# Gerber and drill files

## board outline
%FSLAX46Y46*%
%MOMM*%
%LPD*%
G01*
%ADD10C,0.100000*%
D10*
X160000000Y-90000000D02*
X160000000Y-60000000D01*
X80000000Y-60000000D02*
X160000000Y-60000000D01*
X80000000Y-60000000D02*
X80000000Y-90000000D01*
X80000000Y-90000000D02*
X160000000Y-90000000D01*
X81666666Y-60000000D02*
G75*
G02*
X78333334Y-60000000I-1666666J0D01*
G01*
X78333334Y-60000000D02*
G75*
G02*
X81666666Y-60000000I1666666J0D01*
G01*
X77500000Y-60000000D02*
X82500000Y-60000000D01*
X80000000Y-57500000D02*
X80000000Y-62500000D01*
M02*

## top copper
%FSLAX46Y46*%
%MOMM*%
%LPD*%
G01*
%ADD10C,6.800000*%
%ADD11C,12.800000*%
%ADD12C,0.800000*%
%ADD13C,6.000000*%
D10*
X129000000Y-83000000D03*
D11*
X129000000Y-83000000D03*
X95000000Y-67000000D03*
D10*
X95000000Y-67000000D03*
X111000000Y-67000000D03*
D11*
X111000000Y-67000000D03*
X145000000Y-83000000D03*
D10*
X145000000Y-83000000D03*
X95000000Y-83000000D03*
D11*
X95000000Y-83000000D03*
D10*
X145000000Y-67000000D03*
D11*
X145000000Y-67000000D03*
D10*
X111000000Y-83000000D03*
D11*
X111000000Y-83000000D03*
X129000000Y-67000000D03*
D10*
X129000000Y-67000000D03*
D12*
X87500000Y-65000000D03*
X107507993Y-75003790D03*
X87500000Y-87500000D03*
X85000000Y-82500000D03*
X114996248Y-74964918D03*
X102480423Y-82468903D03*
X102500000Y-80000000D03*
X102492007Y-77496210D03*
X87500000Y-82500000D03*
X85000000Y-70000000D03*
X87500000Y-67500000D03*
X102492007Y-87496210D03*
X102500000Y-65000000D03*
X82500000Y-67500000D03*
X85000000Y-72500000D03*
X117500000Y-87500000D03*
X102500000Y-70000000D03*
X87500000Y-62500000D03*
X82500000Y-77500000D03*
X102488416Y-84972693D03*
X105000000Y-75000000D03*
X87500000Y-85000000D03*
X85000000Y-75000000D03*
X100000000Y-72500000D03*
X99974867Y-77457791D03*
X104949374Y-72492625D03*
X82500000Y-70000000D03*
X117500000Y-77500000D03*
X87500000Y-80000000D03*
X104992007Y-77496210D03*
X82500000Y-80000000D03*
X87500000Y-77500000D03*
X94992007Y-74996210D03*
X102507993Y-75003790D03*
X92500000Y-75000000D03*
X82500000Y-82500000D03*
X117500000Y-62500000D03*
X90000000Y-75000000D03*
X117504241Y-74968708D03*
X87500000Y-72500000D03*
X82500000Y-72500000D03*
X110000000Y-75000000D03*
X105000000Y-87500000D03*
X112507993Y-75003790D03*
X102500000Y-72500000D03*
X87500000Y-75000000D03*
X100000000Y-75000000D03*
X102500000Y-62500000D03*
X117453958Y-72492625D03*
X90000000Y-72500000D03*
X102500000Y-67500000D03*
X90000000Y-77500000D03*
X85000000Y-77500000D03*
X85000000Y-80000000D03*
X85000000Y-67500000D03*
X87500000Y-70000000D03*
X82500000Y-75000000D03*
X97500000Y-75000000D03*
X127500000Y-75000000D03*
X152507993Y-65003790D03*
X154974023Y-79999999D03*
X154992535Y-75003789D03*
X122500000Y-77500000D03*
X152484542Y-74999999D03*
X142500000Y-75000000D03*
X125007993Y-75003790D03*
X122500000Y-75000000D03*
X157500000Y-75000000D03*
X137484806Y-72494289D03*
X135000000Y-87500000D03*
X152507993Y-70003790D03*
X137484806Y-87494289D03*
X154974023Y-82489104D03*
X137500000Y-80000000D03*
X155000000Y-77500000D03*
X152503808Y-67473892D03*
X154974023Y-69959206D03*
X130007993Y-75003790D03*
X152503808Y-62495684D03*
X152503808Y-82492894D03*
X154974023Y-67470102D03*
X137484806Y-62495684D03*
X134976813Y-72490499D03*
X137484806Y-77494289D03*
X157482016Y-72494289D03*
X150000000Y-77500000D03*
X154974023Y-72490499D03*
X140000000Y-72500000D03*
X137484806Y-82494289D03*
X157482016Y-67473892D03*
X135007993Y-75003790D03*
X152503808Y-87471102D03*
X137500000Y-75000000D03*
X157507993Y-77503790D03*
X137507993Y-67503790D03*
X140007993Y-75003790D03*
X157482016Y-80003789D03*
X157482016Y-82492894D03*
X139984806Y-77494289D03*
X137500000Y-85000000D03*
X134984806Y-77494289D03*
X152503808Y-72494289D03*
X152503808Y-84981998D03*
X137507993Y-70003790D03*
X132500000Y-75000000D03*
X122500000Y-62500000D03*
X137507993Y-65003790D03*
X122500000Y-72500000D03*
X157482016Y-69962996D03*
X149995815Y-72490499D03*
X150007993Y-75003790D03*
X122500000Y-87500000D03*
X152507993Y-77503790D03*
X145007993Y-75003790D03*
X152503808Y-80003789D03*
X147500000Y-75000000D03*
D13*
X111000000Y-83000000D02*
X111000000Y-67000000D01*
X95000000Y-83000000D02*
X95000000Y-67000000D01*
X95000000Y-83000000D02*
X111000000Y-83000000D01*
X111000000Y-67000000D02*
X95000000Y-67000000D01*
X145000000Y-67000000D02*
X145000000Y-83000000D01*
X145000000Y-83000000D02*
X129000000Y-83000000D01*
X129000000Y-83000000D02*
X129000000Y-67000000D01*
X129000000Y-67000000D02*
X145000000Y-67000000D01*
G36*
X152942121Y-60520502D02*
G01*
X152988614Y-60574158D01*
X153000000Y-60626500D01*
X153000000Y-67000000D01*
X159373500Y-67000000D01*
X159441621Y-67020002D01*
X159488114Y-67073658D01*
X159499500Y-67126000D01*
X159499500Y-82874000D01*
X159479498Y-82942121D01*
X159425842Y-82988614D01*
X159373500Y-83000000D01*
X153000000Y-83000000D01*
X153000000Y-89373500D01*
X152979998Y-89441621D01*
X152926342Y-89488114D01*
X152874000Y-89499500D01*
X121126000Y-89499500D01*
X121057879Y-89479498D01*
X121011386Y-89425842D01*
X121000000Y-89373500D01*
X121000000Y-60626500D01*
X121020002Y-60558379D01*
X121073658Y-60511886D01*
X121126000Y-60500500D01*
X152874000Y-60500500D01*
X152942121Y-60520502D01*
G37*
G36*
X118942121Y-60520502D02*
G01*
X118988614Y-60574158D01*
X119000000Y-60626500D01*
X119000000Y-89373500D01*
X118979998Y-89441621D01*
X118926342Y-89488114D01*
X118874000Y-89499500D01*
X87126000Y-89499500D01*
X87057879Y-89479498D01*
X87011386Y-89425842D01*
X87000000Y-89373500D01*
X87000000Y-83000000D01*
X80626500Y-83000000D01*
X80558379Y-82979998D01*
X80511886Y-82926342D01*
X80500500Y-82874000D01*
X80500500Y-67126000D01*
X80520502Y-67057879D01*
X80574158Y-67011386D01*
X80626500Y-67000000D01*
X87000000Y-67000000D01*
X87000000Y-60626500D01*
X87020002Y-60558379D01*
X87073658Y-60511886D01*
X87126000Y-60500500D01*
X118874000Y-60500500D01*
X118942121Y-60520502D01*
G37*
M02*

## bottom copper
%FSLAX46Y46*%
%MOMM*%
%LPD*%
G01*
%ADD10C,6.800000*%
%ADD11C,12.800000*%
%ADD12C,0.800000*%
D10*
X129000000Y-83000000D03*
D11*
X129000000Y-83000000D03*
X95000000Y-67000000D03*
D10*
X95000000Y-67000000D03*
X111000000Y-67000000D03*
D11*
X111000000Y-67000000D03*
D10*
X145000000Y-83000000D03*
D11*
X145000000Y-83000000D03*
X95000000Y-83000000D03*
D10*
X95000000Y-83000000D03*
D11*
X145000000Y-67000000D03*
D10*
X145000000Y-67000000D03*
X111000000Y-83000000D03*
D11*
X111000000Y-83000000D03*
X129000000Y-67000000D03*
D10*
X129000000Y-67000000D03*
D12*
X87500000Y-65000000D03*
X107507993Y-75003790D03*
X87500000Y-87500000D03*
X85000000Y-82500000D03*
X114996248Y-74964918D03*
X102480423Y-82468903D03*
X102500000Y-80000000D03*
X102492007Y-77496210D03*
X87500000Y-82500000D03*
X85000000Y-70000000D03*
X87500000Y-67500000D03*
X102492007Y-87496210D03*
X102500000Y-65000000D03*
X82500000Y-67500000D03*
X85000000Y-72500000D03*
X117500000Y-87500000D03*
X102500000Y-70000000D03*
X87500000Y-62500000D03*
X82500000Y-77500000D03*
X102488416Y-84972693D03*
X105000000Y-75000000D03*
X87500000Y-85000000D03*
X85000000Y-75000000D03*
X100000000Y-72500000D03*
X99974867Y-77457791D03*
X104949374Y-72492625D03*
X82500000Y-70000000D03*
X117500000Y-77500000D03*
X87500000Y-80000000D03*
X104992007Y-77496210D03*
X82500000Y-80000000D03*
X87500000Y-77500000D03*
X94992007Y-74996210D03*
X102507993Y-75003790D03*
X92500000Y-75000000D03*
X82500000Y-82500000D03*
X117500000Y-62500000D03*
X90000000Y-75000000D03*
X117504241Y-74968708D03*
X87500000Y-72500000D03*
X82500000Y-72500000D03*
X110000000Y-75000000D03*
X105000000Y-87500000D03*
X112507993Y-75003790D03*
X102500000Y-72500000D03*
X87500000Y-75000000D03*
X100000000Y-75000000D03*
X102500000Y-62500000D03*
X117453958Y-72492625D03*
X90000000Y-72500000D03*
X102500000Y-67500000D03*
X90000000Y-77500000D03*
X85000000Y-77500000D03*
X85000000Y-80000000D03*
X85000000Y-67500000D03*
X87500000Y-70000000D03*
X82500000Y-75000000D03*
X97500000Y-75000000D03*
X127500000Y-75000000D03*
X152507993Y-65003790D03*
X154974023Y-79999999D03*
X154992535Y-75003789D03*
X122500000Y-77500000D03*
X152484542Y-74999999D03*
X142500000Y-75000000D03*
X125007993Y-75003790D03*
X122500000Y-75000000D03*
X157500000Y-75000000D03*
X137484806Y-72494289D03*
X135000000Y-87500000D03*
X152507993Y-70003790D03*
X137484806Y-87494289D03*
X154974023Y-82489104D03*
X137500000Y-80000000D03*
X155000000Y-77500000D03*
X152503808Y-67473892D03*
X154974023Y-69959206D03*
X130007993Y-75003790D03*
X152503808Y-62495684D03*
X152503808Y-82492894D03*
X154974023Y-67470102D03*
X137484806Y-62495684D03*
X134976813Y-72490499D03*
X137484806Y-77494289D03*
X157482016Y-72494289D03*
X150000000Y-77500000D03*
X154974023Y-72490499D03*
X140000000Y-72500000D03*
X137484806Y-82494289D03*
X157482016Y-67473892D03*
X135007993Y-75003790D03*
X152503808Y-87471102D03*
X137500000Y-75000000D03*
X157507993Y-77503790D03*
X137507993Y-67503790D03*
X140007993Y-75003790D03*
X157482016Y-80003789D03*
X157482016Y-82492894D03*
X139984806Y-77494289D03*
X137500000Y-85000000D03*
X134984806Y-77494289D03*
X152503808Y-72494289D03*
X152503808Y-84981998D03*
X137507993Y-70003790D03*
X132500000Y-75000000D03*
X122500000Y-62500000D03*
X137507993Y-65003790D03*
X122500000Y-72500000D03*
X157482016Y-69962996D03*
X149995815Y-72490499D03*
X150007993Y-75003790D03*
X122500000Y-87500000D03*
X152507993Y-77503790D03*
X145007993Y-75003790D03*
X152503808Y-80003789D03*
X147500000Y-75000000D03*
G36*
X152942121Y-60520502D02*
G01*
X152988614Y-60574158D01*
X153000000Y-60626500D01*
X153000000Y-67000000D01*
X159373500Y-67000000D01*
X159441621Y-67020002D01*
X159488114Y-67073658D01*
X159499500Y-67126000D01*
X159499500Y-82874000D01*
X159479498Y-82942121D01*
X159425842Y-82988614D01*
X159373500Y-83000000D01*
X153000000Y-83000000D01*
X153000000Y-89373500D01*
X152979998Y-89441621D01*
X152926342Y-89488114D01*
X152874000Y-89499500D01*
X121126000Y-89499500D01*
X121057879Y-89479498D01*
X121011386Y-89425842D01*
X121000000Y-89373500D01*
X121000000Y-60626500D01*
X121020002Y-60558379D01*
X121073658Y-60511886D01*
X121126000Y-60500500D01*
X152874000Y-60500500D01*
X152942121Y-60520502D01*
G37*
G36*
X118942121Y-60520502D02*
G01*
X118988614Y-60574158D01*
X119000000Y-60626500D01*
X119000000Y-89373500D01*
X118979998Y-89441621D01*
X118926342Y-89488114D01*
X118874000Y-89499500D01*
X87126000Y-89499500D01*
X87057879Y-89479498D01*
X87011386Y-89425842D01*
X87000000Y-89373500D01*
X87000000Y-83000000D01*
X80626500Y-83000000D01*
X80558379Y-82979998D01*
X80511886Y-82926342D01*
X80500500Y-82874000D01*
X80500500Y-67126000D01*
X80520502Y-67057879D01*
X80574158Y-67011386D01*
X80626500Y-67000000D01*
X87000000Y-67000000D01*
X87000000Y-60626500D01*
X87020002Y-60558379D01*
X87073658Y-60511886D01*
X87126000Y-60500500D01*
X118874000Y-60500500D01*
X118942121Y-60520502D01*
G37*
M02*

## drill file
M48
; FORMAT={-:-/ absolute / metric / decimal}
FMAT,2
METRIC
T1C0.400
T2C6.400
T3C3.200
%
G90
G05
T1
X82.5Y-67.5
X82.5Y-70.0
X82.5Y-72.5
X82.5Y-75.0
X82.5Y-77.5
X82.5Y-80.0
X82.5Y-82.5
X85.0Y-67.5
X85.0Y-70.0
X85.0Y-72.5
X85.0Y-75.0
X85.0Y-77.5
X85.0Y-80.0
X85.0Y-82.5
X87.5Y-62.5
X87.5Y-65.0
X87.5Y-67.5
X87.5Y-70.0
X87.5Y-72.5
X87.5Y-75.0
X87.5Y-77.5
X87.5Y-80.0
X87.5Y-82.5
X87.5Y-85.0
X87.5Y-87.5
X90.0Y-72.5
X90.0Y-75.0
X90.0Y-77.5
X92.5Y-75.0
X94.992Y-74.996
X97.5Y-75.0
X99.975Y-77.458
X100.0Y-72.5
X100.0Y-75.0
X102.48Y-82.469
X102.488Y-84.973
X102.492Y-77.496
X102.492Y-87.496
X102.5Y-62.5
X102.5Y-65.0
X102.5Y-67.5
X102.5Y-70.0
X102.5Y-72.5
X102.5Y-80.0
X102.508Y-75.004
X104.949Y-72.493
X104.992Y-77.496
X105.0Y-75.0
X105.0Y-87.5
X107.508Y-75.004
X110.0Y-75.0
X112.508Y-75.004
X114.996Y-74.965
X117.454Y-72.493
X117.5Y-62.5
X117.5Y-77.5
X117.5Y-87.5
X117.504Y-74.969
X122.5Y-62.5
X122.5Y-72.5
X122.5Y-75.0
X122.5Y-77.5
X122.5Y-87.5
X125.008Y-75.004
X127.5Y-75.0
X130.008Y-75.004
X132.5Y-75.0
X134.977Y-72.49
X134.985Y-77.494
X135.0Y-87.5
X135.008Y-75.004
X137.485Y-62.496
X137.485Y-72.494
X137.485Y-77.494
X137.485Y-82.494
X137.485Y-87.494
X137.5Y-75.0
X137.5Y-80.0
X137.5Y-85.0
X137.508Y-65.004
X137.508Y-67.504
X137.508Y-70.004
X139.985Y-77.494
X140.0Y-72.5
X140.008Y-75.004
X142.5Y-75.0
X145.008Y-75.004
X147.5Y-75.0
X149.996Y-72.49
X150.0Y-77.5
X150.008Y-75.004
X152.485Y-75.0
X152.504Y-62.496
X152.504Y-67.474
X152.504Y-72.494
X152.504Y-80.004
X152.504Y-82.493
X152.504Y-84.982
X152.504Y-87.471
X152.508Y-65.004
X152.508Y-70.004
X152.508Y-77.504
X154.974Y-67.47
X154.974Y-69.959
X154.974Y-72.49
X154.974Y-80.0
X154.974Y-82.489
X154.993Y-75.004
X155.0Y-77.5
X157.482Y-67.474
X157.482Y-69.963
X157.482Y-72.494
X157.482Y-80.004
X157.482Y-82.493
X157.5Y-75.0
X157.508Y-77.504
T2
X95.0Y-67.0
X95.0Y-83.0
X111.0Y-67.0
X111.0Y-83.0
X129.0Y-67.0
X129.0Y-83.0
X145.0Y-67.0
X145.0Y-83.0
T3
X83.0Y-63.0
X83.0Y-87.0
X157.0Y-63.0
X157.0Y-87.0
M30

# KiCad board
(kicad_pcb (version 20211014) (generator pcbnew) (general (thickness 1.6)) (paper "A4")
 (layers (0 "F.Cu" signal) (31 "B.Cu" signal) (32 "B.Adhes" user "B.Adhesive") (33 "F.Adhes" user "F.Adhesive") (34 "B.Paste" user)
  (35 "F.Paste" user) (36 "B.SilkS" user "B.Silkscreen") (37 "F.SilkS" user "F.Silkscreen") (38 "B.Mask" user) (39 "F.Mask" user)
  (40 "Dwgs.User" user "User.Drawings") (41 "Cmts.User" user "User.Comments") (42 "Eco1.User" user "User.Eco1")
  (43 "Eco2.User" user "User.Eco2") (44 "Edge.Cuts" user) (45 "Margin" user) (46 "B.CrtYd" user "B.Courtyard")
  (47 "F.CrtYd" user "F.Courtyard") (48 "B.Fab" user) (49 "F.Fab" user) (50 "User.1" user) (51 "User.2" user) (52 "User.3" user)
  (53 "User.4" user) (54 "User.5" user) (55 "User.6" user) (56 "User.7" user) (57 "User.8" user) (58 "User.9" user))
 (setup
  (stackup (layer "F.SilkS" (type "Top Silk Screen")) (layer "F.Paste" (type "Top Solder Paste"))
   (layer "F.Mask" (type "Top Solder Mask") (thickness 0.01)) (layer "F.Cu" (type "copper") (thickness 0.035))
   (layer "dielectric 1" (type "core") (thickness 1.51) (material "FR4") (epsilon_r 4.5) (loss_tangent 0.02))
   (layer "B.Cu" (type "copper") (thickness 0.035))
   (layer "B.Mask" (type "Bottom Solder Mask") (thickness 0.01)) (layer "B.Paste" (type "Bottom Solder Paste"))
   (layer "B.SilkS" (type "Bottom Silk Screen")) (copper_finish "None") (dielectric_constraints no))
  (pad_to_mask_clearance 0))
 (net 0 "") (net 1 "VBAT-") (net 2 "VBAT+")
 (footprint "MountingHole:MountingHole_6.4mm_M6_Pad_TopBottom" (layer "F.Cu") (at 129 83 90)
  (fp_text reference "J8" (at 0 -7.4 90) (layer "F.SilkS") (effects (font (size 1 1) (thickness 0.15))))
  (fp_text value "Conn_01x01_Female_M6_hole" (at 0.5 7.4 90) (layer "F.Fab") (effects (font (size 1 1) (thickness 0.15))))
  (pad "1" thru_hole circle locked (at 0 0 90) (size 6.8 6.8) (drill 6.4) (layers *.Cu *.Mask) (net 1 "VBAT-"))
  (pad "1" connect circle locked (at 0 0 90) (size 12.8 12.8) (layers "F.Cu" "F.Mask") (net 1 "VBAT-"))
  (pad "1" connect circle locked (at 0 0 90) (size 12.8 12.8) (layers "B.Cu" "B.Mask") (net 1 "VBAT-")))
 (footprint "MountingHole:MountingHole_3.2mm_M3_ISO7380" (layer "F.Cu") (at 157 87)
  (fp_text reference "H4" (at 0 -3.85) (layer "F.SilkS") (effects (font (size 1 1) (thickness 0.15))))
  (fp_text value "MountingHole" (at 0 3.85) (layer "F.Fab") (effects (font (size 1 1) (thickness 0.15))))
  (pad "" np_thru_hole circle locked (at 0 0) (size 3.2 3.2) (drill 3.2) (layers *.Cu *.Mask)))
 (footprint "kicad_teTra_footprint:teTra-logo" (layer "F.Cu") (at 85 74 -90)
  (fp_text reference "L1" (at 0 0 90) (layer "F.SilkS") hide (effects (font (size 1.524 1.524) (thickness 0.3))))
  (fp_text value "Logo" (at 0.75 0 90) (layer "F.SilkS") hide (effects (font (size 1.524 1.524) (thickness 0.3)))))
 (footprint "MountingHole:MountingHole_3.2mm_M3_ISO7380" (layer "F.Cu") (at 83 87)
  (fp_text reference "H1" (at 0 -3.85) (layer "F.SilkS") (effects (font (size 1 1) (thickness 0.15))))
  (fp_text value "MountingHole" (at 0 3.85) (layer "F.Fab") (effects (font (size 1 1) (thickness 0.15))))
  (pad "" np_thru_hole circle locked (at 0 0) (size 3.2 3.2) (drill 3.2) (layers *.Cu *.Mask)))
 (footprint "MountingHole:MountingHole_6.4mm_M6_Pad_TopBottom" (layer "F.Cu") (at 95 67 90)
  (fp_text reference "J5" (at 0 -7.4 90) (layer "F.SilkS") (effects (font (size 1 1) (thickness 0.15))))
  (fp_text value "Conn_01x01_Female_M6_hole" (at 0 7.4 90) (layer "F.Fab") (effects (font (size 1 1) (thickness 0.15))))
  (pad "1" connect circle locked (at 0 0 90) (size 12.8 12.8) (layers "B.Cu" "B.Mask") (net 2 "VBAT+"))
  (pad "1" connect circle locked (at 0 0 90) (size 12.8 12.8) (layers "F.Cu" "F.Mask") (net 2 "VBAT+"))
  (pad "1" thru_hole circle locked (at 0 0 90) (size 6.8 6.8) (drill 6.4) (layers *.Cu *.Mask) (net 2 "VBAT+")))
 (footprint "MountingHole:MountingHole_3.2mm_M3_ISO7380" (layer "F.Cu") (at 83 63)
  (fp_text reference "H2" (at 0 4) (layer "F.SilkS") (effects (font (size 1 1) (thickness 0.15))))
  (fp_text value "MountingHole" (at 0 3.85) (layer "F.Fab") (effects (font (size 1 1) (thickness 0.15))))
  (pad "" np_thru_hole circle locked (at 0 0) (size 3.2 3.2) (drill 3.2) (layers *.Cu *.Mask)))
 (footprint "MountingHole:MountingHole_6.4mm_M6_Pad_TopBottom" (layer "F.Cu") (at 111 67 90)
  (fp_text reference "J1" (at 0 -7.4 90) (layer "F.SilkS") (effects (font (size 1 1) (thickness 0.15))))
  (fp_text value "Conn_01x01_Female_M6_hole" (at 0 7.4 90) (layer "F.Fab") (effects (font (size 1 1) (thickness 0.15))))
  (pad "1" thru_hole circle locked (at 0 0 90) (size 6.8 6.8) (drill 6.4) (layers *.Cu *.Mask) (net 2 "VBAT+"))
  (pad "1" connect circle locked (at 0 0 90) (size 12.8 12.8) (layers "F.Cu" "F.Mask") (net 2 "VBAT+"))
  (pad "1" connect circle locked (at 0 0 90) (size 12.8 12.8) (layers "B.Cu" "B.Mask") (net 2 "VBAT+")))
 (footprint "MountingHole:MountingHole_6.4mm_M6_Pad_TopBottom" (layer "F.Cu") (at 145 83 90)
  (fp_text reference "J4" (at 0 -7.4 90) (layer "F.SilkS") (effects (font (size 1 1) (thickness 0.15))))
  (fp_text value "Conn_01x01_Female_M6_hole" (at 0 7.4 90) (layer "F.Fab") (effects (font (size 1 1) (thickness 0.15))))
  (pad "1" connect circle locked (at 0 0 90) (size 12.8 12.8) (layers "F.Cu" "F.Mask") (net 1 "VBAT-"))
  (pad "1" thru_hole circle locked (at 0 0 90) (size 6.8 6.8) (drill 6.4) (layers *.Cu *.Mask) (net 1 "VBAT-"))
  (pad "1" connect circle locked (at 0 0 90) (size 12.8 12.8) (layers "B.Cu" "B.Mask") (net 1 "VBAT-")))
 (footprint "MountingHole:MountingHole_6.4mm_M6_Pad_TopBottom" (layer "F.Cu") (at 95 83 90)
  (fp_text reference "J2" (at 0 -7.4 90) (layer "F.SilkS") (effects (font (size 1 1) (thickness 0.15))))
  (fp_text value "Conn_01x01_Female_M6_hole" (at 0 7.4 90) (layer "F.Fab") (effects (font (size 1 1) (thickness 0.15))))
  (pad "1" connect circle locked (at 0 0 90) (size 12.8 12.8) (layers "B.Cu" "B.Mask") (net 2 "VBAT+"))
  (pad "1" thru_hole circle locked (at 0 0 90) (size 6.8 6.8) (drill 6.4) (layers *.Cu *.Mask) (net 2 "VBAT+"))
  (pad "1" connect circle locked (at 0 0 90) (size 12.8 12.8) (layers "F.Cu" "F.Mask") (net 2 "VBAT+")))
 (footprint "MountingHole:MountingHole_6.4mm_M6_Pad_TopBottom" (layer "F.Cu") (at 145 67 90)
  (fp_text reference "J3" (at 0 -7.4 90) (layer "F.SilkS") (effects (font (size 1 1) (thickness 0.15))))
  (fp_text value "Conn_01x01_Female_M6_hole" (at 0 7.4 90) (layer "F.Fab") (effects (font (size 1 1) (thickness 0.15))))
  (pad "1" connect circle locked (at 0 0 90) (size 12.8 12.8) (layers "B.Cu" "B.Mask") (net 1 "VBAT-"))
  (pad "1" thru_hole circle locked (at 0 0 90) (size 6.8 6.8) (drill 6.4) (layers *.Cu *.Mask) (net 1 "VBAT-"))
  (pad "1" connect circle locked (at 0 0 90) (size 12.8 12.8) (layers "F.Cu" "F.Mask") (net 1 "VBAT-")))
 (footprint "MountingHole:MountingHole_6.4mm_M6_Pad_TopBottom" (layer "F.Cu") (at 111 83 90)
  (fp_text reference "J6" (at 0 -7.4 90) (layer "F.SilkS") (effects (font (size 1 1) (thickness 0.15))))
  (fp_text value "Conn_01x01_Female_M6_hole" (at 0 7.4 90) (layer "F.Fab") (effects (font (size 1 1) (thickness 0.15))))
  (pad "1" thru_hole circle locked (at 0 0 90) (size 6.8 6.8) (drill 6.4) (layers *.Cu *.Mask) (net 2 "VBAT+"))
  (pad "1" connect circle locked (at 0 0 90) (size 12.8 12.8) (layers "B.Cu" "B.Mask") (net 2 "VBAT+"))
  (pad "1" connect circle locked (at 0 0 90) (size 12.8 12.8) (layers "F.Cu" "F.Mask") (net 2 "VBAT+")))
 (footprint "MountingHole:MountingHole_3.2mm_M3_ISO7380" (layer "F.Cu") (at 157 63)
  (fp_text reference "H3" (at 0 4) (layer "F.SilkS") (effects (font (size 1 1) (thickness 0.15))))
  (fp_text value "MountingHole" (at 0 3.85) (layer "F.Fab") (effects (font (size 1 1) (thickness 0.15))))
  (pad "" np_thru_hole circle locked (at 0 0) (size 3.2 3.2) (drill 3.2) (layers *.Cu *.Mask)))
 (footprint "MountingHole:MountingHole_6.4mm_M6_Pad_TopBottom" (layer "F.Cu") (at 129 67 90)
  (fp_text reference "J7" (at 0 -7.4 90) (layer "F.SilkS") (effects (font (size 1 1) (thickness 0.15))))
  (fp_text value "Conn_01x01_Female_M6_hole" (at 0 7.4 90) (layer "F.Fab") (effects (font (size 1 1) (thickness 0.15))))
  (pad "1" connect circle locked (at 0 0 90) (size 12.8 12.8) (layers "F.Cu" "F.Mask") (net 1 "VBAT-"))
  (pad "1" connect circle locked (at 0 0 90) (size 12.8 12.8) (layers "B.Cu" "B.Mask") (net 1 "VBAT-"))
  (pad "1" thru_hole circle locked (at 0 0 90) (size 6.8 6.8) (drill 6.4) (layers *.Cu *.Mask) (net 1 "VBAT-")))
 (gr_line (start 160 90) (end 160 60) (layer "Edge.Cuts") (width 0.1))
 (gr_line (start 80 60) (end 160 60) (layer "Edge.Cuts") (width 0.1))
 (gr_line (start 80 60) (end 80 90) (layer "Edge.Cuts") (width 0.1))
 (gr_line (start 80 90) (end 160 90) (layer "Edge.Cuts") (width 0.1))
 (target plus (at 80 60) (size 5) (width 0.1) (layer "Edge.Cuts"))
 (segment (start 111 83) (end 111 67) (width 6) (layer "F.Cu") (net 2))
 (segment (start 95 83) (end 95 67) (width 6) (layer "F.Cu") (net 2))
 (segment (start 95 83) (end 111 83) (width 6) (layer "F.Cu") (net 2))
 (segment (start 111 67) (end 95 67) (width 6) (layer "F.Cu") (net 2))
 (via (at 87.5 65) (size 0.8) (drill 0.4) (layers "F.Cu" "B.Cu") (free) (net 2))
 (via (at 107.507993 75.00379) (size 0.8) (drill 0.4) (layers "F.Cu" "B.Cu") (free) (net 2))
 (via (at 87.5 87.5) (size 0.8) (drill 0.4) (layers "F.Cu" "B.Cu") (free) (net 2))
 (via (at 85 82.5) (size 0.8) (drill 0.4) (layers "F.Cu" "B.Cu") (free) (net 2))
 (via (at 114.996248 74.964918) (size 0.8) (drill 0.4) (layers "F.Cu" "B.Cu") (free) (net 2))
 (via (at 102.480423 82.468903) (size 0.8) (drill 0.4) (layers "F.Cu" "B.Cu") (free) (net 2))
 (via (at 102.5 80) (size 0.8) (drill 0.4) (layers "F.Cu" "B.Cu") (free) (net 2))
 (via (at 102.492007 77.49621) (size 0.8) (drill 0.4) (layers "F.Cu" "B.Cu") (free) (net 2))
 (via (at 87.5 82.5) (size 0.8) (drill 0.4) (layers "F.Cu" "B.Cu") (free) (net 2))
 (via (at 85 70) (size 0.8) (drill 0.4) (layers "F.Cu" "B.Cu") (free) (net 2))
 (via (at 87.5 67.5) (size 0.8) (drill 0.4) (layers "F.Cu" "B.Cu") (free) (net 2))
 (via (at 102.492007 87.49621) (size 0.8) (drill 0.4) (layers "F.Cu" "B.Cu") (free) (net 2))
 (via (at 102.5 65) (size 0.8) (drill 0.4) (layers "F.Cu" "B.Cu") (free) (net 2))
 (via (at 82.5 67.5) (size 0.8) (drill 0.4) (layers "F.Cu" "B.Cu") (free) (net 2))
 (via (at 85 72.5) (size 0.8) (drill 0.4) (layers "F.Cu" "B.Cu") (free) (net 2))
 (via (at 117.5 87.5) (size 0.8) (drill 0.4) (layers "F.Cu" "B.Cu") (free) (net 2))
 (via (at 102.5 70) (size 0.8) (drill 0.4) (layers "F.Cu" "B.Cu") (free) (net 2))
 (via (at 87.5 62.5) (size 0.8) (drill 0.4) (layers "F.Cu" "B.Cu") (free) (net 2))
 (via (at 82.5 77.5) (size 0.8) (drill 0.4) (layers "F.Cu" "B.Cu") (free) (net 2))
 (via (at 102.488416 84.972693) (size 0.8) (drill 0.4) (layers "F.Cu" "B.Cu") (free) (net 2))
 (via (at 105 75) (size 0.8) (drill 0.4) (layers "F.Cu" "B.Cu") (free) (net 2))
 (via (at 87.5 85) (size 0.8) (drill 0.4) (layers "F.Cu" "B.Cu") (free) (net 2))
 (via (at 85 75) (size 0.8) (drill 0.4) (layers "F.Cu" "B.Cu") (free) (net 2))
 (via (at 100 72.5) (size 0.8) (drill 0.4) (layers "F.Cu" "B.Cu") (free) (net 2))
 (via (at 99.974867 77.457791) (size 0.8) (drill 0.4) (layers "F.Cu" "B.Cu") (free) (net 2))
 (via (at 104.949374 72.492625) (size 0.8) (drill 0.4) (layers "F.Cu" "B.Cu") (free) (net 2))
 (via (at 82.5 70) (size 0.8) (drill 0.4) (layers "F.Cu" "B.Cu") (free) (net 2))
 (via (at 117.5 77.5) (size 0.8) (drill 0.4) (layers "F.Cu" "B.Cu") (free) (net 2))
 (via (at 87.5 80) (size 0.8) (drill 0.4) (layers "F.Cu" "B.Cu") (free) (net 2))
 (via (at 104.992007 77.49621) (size 0.8) (drill 0.4) (layers "F.Cu" "B.Cu") (free) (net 2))
 (via (at 82.5 80) (size 0.8) (drill 0.4) (layers "F.Cu" "B.Cu") (free) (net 2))
 (via (at 87.5 77.5) (size 0.8) (drill 0.4) (layers "F.Cu" "B.Cu") (free) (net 2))
 (via (at 94.992007 74.99621) (size 0.8) (drill 0.4) (layers "F.Cu" "B.Cu") (free) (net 2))
 (via (at 102.507993 75.00379) (size 0.8) (drill 0.4) (layers "F.Cu" "B.Cu") (free) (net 2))
 (via (at 92.5 75) (size 0.8) (drill 0.4) (layers "F.Cu" "B.Cu") (free) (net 2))
 (via (at 82.5 82.5) (size 0.8) (drill 0.4) (layers "F.Cu" "B.Cu") (free) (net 2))
 (via (at 117.5 62.5) (size 0.8) (drill 0.4) (layers "F.Cu" "B.Cu") (free) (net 2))
 (via (at 90 75) (size 0.8) (drill 0.4) (layers "F.Cu" "B.Cu") (free) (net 2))
 (via (at 117.504241 74.968708) (size 0.8) (drill 0.4) (layers "F.Cu" "B.Cu") (free) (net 2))
 (via (at 87.5 72.5) (size 0.8) (drill 0.4) (layers "F.Cu" "B.Cu") (free) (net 2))
 (via (at 82.5 72.5) (size 0.8) (drill 0.4) (layers "F.Cu" "B.Cu") (free) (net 2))
 (via (at 110 75) (size 0.8) (drill 0.4) (layers "F.Cu" "B.Cu") (free) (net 2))
 (via (at 105 87.5) (size 0.8) (drill 0.4) (layers "F.Cu" "B.Cu") (free) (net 2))
 (via (at 112.507993 75.00379) (size 0.8) (drill 0.4) (layers "F.Cu" "B.Cu") (free) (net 2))
 (via (at 102.5 72.5) (size 0.8) (drill 0.4) (layers "F.Cu" "B.Cu") (free) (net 2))
 (via (at 87.5 75) (size 0.8) (drill 0.4) (layers "F.Cu" "B.Cu") (free) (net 2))
 (via (at 100 75) (size 0.8) (drill 0.4) (layers "F.Cu" "B.Cu") (free) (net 2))
 (via (at 102.5 62.5) (size 0.8) (drill 0.4) (layers "F.Cu" "B.Cu") (free) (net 2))
 (via (at 117.453958 72.492625) (size 0.8) (drill 0.4) (layers "F.Cu" "B.Cu") (free) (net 2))
 (via (at 90 72.5) (size 0.8) (drill 0.4) (layers "F.Cu" "B.Cu") (free) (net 2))
 (via (at 102.5 67.5) (size 0.8) (drill 0.4) (layers "F.Cu" "B.Cu") (free) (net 2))
 (via (at 90 77.5) (size 0.8) (drill 0.4) (layers "F.Cu" "B.Cu") (free) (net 2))
 (via (at 85 77.5) (size 0.8) (drill 0.4) (layers "F.Cu" "B.Cu") (free) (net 2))
 (via (at 85 80) (size 0.8) (drill 0.4) (layers "F.Cu" "B.Cu") (free) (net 2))
 (via (at 85 67.5) (size 0.8) (drill 0.4) (layers "F.Cu" "B.Cu") (free) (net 2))
 (via (at 87.5 70) (size 0.8) (drill 0.4) (layers "F.Cu" "B.Cu") (free) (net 2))
 (via (at 82.5 75) (size 0.8) (drill 0.4) (layers "F.Cu" "B.Cu") (free) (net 2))
 (via (at 97.5 75) (size 0.8) (drill 0.4) (layers "F.Cu" "B.Cu") (free) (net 2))
 (segment (start 145 67) (end 145 83) (width 6) (layer "F.Cu") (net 1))
 (segment (start 145 83) (end 129 83) (width 6) (layer "F.Cu") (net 1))
 (segment (start 129 83) (end 129 67) (width 6) (layer "F.Cu") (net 1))
 (segment (start 129 67) (end 145 67) (width 6) (layer "F.Cu") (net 1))
 (via (at 127.5 75) (size 0.8) (drill 0.4) (layers "F.Cu" "B.Cu") (free) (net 1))
 (via (at 152.507993 65.00379) (size 0.8) (drill 0.4) (layers "F.Cu" "B.Cu") (free) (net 1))
 (via (at 154.974023 79.999999) (size 0.8) (drill 0.4) (layers "F.Cu" "B.Cu") (free) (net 1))
 (via (at 154.992535 75.003789) (size 0.8) (drill 0.4) (layers "F.Cu" "B.Cu") (free) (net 1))
 (via (at 122.5 77.5) (size 0.8) (drill 0.4) (layers "F.Cu" "B.Cu") (free) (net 1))
 (via (at 152.484542 74.999999) (size 0.8) (drill 0.4) (layers "F.Cu" "B.Cu") (free) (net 1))
 (via (at 142.5 75) (size 0.8) (drill 0.4) (layers "F.Cu" "B.Cu") (free) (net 1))
 (via (at 125.007993 75.00379) (size 0.8) (drill 0.4) (layers "F.Cu" "B.Cu") (free) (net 1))
 (via (at 122.5 75) (size 0.8) (drill 0.4) (layers "F.Cu" "B.Cu") (free) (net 1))
 (via (at 157.5 75) (size 0.8) (drill 0.4) (layers "F.Cu" "B.Cu") (free) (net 1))
 (via (at 137.484806 72.494289) (size 0.8) (drill 0.4) (layers "F.Cu" "B.Cu") (free) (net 1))
 (via (at 135 87.5) (size 0.8) (drill 0.4) (layers "F.Cu" "B.Cu") (free) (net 1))
 (via (at 152.507993 70.00379) (size 0.8) (drill 0.4) (layers "F.Cu" "B.Cu") (free) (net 1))
 (via (at 137.484806 87.494289) (size 0.8) (drill 0.4) (layers "F.Cu" "B.Cu") (free) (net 1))
 (via (at 154.974023 82.489104) (size 0.8) (drill 0.4) (layers "F.Cu" "B.Cu") (free) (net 1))
 (via (at 137.5 80) (size 0.8) (drill 0.4) (layers "F.Cu" "B.Cu") (free) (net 1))
 (via (at 155 77.5) (size 0.8) (drill 0.4) (layers "F.Cu" "B.Cu") (free) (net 1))
 (via (at 152.503808 67.473892) (size 0.8) (drill 0.4) (layers "F.Cu" "B.Cu") (free) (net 1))
 (via (at 154.974023 69.959206) (size 0.8) (drill 0.4) (layers "F.Cu" "B.Cu") (free) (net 1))
 (via (at 130.007993 75.00379) (size 0.8) (drill 0.4) (layers "F.Cu" "B.Cu") (free) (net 1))
 (via (at 152.503808 62.495684) (size 0.8) (drill 0.4) (layers "F.Cu" "B.Cu") (free) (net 1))
 (via (at 152.503808 82.492894) (size 0.8) (drill 0.4) (layers "F.Cu" "B.Cu") (free) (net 1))
 (via (at 154.974023 67.470102) (size 0.8) (drill 0.4) (layers "F.Cu" "B.Cu") (free) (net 1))
 (via (at 137.484806 62.495684) (size 0.8) (drill 0.4) (layers "F.Cu" "B.Cu") (free) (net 1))
 (via (at 134.976813 72.490499) (size 0.8) (drill 0.4) (layers "F.Cu" "B.Cu") (free) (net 1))
 (via (at 137.484806 77.494289) (size 0.8) (drill 0.4) (layers "F.Cu" "B.Cu") (free) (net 1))
 (via (at 157.482016 72.494289) (size 0.8) (drill 0.4) (layers "F.Cu" "B.Cu") (free) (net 1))
 (via (at 150 77.5) (size 0.8) (drill 0.4) (layers "F.Cu" "B.Cu") (free) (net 1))
 (via (at 154.974023 72.490499) (size 0.8) (drill 0.4) (layers "F.Cu" "B.Cu") (free) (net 1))
 (via (at 140 72.5) (size 0.8) (drill 0.4) (layers "F.Cu" "B.Cu") (free) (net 1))
 (via (at 137.484806 82.494289) (size 0.8) (drill 0.4) (layers "F.Cu" "B.Cu") (free) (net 1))
 (via (at 157.482016 67.473892) (size 0.8) (drill 0.4) (layers "F.Cu" "B.Cu") (free) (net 1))
 (via (at 135.007993 75.00379) (size 0.8) (drill 0.4) (layers "F.Cu" "B.Cu") (free) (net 1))
 (via (at 152.503808 87.471102) (size 0.8) (drill 0.4) (layers "F.Cu" "B.Cu") (free) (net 1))
 (via (at 137.5 75) (size 0.8) (drill 0.4) (layers "F.Cu" "B.Cu") (free) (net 1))
 (via (at 157.507993 77.50379) (size 0.8) (drill 0.4) (layers "F.Cu" "B.Cu") (free) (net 1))
 (via (at 137.507993 67.50379) (size 0.8) (drill 0.4) (layers "F.Cu" "B.Cu") (free) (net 1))
 (via (at 140.007993 75.00379) (size 0.8) (drill 0.4) (layers "F.Cu" "B.Cu") (free) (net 1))
 (via (at 157.482016 80.003789) (size 0.8) (drill 0.4) (layers "F.Cu" "B.Cu") (free) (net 1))
 (via (at 157.482016 82.492894) (size 0.8) (drill 0.4) (layers "F.Cu" "B.Cu") (free) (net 1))
 (via (at 139.984806 77.494289) (size 0.8) (drill 0.4) (layers "F.Cu" "B.Cu") (free) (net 1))
 (via (at 137.5 85) (size 0.8) (drill 0.4) (layers "F.Cu" "B.Cu") (free) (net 1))
 (via (at 134.984806 77.494289) (size 0.8) (drill 0.4) (layers "F.Cu" "B.Cu") (free) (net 1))
 (via (at 152.503808 72.494289) (size 0.8) (drill 0.4) (layers "F.Cu" "B.Cu") (free) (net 1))
 (via (at 152.503808 84.981998) (size 0.8) (drill 0.4) (layers "F.Cu" "B.Cu") (free) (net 1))
 (via (at 137.507993 70.00379) (size 0.8) (drill 0.4) (layers "F.Cu" "B.Cu") (free) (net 1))
 (via (at 132.5 75) (size 0.8) (drill 0.4) (layers "F.Cu" "B.Cu") (free) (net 1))
 (via (at 122.5 62.5) (size 0.8) (drill 0.4) (layers "F.Cu" "B.Cu") (free) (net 1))
 (via (at 137.507993 65.00379) (size 0.8) (drill 0.4) (layers "F.Cu" "B.Cu") (free) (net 1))
 (via (at 122.5 72.5) (size 0.8) (drill 0.4) (layers "F.Cu" "B.Cu") (free) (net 1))
 (via (at 157.482016 69.962996) (size 0.8) (drill 0.4) (layers "F.Cu" "B.Cu") (free) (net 1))
 (via (at 149.995815 72.490499) (size 0.8) (drill 0.4) (layers "F.Cu" "B.Cu") (free) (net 1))
 (via (at 150.007993 75.00379) (size 0.8) (drill 0.4) (layers "F.Cu" "B.Cu") (free) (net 1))
 (via (at 122.5 87.5) (size 0.8) (drill 0.4) (layers "F.Cu" "B.Cu") (free) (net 1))
 (via (at 152.507993 77.50379) (size 0.8) (drill 0.4) (layers "F.Cu" "B.Cu") (free) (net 1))
 (via (at 145.007993 75.00379) (size 0.8) (drill 0.4) (layers "F.Cu" "B.Cu") (free) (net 1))
 (via (at 152.503808 80.003789) (size 0.8) (drill 0.4) (layers "F.Cu" "B.Cu") (free) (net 1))
 (via (at 147.5 75) (size 0.8) (drill 0.4) (layers "F.Cu" "B.Cu") (free) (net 1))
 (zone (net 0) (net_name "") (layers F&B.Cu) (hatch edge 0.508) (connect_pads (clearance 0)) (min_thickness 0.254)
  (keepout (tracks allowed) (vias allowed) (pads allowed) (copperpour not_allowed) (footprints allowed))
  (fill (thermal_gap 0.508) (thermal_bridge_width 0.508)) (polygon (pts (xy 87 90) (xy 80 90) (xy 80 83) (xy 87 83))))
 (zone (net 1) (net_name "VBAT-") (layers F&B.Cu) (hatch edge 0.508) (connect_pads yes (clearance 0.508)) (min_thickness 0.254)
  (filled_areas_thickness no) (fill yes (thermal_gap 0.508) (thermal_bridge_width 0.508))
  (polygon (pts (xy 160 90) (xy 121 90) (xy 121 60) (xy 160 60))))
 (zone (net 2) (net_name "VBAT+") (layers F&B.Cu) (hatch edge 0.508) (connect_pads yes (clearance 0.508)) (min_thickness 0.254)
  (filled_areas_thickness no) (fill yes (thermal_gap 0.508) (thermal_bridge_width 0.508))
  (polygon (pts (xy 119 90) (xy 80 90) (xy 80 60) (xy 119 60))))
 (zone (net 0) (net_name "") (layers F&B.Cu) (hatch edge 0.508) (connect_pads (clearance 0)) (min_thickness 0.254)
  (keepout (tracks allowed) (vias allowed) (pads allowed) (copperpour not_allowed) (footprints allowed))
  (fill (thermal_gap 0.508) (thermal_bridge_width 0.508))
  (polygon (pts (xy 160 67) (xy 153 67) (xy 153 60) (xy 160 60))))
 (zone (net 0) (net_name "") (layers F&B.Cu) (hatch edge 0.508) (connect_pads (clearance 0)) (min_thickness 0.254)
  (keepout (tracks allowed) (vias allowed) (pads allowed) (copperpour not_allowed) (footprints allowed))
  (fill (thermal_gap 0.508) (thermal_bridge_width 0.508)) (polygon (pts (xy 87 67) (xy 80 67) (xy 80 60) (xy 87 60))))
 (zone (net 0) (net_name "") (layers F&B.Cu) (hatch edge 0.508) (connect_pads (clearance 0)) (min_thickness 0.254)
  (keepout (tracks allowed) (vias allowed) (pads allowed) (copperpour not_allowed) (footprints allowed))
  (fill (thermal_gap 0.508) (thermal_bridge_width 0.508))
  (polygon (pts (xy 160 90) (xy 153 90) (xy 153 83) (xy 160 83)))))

